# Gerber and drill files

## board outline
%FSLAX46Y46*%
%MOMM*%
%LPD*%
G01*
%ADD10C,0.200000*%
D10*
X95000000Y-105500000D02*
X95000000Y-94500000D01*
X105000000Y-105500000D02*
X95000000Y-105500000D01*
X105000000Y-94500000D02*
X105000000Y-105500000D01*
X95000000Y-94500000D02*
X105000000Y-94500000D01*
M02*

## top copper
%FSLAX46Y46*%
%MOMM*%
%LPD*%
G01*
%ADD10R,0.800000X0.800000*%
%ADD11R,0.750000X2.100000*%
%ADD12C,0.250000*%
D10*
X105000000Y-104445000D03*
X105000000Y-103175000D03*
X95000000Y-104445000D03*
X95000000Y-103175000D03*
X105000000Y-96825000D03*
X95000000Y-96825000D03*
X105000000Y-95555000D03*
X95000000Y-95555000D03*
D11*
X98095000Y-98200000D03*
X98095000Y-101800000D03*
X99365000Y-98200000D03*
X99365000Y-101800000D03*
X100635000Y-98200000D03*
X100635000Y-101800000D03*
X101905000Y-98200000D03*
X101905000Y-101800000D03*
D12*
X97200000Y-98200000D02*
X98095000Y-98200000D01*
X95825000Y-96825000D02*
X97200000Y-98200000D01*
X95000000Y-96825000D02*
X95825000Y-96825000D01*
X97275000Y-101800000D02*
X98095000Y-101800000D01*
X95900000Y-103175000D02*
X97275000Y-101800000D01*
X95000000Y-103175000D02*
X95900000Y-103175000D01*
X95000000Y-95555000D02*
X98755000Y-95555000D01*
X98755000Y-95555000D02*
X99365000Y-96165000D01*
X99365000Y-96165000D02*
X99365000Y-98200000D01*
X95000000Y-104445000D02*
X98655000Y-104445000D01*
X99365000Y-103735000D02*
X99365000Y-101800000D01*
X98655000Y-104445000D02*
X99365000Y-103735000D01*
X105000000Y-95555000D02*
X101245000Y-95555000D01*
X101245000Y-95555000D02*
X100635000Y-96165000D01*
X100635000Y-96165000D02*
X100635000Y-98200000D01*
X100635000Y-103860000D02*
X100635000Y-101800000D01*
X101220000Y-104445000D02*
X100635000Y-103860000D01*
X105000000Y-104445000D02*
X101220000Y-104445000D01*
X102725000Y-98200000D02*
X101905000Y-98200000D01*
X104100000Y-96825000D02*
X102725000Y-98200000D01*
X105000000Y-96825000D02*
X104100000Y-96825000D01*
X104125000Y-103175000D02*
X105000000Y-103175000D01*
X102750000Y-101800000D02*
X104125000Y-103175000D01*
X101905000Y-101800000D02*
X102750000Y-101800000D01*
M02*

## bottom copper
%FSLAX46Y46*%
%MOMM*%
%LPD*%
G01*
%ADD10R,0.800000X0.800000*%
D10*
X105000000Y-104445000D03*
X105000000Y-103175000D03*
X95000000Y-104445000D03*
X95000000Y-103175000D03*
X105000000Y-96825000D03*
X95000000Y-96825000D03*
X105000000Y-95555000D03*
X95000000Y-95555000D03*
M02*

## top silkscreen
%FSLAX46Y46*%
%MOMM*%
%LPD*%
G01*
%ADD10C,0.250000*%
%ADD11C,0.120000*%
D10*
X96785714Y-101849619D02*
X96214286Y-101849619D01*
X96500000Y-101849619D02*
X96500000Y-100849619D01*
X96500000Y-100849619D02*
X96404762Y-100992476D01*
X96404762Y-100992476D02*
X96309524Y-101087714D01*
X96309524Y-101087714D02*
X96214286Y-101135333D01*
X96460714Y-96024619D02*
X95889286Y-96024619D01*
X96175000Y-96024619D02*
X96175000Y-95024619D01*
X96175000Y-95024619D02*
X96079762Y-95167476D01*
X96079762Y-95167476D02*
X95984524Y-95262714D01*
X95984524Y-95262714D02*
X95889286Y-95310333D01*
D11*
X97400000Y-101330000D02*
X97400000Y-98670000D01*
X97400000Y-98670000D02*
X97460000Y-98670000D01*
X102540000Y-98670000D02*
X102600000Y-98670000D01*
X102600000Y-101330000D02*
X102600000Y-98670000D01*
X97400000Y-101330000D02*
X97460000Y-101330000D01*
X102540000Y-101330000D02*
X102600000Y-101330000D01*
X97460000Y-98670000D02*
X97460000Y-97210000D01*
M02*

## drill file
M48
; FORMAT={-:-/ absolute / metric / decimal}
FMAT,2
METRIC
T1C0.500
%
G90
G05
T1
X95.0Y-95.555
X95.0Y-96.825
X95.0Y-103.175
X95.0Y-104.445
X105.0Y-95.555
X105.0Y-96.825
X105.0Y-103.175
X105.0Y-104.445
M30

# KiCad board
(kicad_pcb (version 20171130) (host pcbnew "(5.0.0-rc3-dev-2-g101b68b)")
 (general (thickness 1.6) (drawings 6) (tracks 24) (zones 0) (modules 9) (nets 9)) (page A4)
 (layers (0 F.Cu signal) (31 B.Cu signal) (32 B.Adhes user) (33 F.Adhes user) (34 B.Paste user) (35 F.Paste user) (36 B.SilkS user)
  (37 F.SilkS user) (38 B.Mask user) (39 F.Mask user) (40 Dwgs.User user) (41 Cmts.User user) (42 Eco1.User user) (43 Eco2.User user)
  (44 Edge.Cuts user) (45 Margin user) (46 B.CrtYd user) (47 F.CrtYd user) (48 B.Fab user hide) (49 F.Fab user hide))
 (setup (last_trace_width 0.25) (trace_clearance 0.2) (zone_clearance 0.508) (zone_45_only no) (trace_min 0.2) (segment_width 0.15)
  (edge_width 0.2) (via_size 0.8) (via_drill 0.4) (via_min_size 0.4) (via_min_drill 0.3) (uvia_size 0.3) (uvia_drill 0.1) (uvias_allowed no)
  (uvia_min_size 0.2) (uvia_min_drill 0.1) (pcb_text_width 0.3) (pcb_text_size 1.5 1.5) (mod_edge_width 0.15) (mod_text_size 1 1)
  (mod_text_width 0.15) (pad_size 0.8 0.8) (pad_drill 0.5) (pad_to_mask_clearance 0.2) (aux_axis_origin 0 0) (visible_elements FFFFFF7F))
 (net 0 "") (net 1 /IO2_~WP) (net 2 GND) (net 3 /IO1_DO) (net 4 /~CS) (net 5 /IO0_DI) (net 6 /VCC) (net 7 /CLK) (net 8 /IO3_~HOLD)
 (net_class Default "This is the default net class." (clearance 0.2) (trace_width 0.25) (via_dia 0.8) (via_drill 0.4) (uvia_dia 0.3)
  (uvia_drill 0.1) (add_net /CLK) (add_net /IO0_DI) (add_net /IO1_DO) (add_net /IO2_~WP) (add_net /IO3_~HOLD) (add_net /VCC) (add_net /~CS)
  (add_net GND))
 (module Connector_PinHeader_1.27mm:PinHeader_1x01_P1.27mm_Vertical (layer F.Cu) (at 105 104.445)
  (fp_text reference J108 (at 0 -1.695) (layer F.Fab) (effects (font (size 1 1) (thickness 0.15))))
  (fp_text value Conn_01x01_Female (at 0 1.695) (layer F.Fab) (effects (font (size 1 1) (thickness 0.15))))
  (pad 1 thru_hole rect (at 0 0) (size 0.8 0.8) (drill 0.5) (layers *.Cu *.Mask) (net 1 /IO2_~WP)))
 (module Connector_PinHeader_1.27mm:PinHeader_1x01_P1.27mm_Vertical (layer F.Cu) (at 105 103.175)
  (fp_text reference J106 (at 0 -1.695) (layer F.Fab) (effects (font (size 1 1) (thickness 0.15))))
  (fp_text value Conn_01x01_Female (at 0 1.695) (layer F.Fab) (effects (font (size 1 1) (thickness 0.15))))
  (pad 1 thru_hole rect (at 0 0) (size 0.8 0.8) (drill 0.5) (layers *.Cu *.Mask) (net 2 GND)))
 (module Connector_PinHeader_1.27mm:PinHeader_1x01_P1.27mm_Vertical (layer F.Cu) (at 95 104.445)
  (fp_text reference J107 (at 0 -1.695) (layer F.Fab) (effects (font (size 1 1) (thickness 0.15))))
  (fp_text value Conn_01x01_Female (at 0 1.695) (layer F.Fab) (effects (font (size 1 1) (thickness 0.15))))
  (pad 1 thru_hole rect (at 0 0) (size 0.8 0.8) (drill 0.5) (layers *.Cu *.Mask) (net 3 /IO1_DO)))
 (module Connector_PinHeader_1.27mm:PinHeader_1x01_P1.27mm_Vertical (layer F.Cu) (at 95 103.175)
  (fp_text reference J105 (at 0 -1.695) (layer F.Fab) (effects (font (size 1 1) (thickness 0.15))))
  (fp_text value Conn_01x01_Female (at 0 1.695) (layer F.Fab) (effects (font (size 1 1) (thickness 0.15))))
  (pad 1 thru_hole rect (at 0 0) (size 0.8 0.8) (drill 0.5) (layers *.Cu *.Mask) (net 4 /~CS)))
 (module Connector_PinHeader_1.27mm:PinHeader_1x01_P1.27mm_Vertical (layer F.Cu) (at 105 96.825)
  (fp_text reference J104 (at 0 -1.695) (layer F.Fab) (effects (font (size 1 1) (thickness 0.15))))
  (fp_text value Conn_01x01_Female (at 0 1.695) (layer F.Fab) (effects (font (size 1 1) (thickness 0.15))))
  (pad 1 thru_hole rect (at 0 0) (size 0.8 0.8) (drill 0.5) (layers *.Cu *.Mask) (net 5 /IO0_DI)))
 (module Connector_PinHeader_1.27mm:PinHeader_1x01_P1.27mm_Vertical (layer F.Cu) (at 95 96.825)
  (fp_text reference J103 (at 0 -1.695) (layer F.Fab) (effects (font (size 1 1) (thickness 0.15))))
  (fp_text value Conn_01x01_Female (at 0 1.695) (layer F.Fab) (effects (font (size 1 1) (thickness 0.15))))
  (pad 1 thru_hole rect (at 0 0) (size 0.8 0.8) (drill 0.5) (layers *.Cu *.Mask) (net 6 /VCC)))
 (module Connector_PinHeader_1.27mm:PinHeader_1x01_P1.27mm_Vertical (layer F.Cu) (at 105 95.555)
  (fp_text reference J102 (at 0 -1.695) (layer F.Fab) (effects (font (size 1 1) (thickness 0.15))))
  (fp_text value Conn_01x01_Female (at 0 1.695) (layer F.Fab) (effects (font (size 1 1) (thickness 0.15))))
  (pad 1 thru_hole rect (at 0 0) (size 0.8 0.8) (drill 0.5) (layers *.Cu *.Mask) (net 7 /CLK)))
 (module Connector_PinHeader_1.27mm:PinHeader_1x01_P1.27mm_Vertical (layer F.Cu) (at 95 95.555)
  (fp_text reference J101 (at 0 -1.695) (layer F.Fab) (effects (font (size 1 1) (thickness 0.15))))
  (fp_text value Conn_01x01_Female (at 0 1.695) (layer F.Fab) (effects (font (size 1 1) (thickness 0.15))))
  (pad 1 thru_hole rect (at 0 0) (size 0.8 0.8) (drill 0.5) (layers *.Cu *.Mask) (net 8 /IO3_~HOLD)))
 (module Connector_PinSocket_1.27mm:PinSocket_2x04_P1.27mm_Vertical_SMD (layer F.Cu) (at 100 100 90)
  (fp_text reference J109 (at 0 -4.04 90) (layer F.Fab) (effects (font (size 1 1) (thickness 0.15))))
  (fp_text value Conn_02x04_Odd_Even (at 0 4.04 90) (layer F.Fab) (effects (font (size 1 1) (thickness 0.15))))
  (fp_line (start -1.33 -2.6) (end 1.33 -2.6) (layer F.SilkS) (width 0.12))
  (fp_line (start 1.33 -2.6) (end 1.33 -2.54) (layer F.SilkS) (width 0.12))
  (fp_line (start 1.33 2.54) (end 1.33 2.6) (layer F.SilkS) (width 0.12))
  (fp_line (start -1.33 2.6) (end 1.33 2.6) (layer F.SilkS) (width 0.12))
  (fp_line (start -1.33 -2.6) (end -1.33 -2.54) (layer F.SilkS) (width 0.12))
  (fp_line (start -1.33 2.54) (end -1.33 2.6) (layer F.SilkS) (width 0.12))
  (fp_line (start 1.33 -2.54) (end 2.79 -2.54) (layer F.SilkS) (width 0.12))
  (pad 1 smd rect (at 1.8 -1.905 90) (size 2.1 0.75) (layers F.Cu F.Paste F.Mask) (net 6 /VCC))
  (pad 2 smd rect (at -1.8 -1.905 90) (size 2.1 0.75) (layers F.Cu F.Paste F.Mask) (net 4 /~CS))
  (pad 3 smd rect (at 1.8 -0.635 90) (size 2.1 0.75) (layers F.Cu F.Paste F.Mask) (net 8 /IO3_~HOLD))
  (pad 4 smd rect (at -1.8 -0.635 90) (size 2.1 0.75) (layers F.Cu F.Paste F.Mask) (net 3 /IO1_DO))
  (pad 5 smd rect (at 1.8 0.635 90) (size 2.1 0.75) (layers F.Cu F.Paste F.Mask) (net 7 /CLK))
  (pad 6 smd rect (at -1.8 0.635 90) (size 2.1 0.75) (layers F.Cu F.Paste F.Mask) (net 1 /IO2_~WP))
  (pad 7 smd rect (at 1.8 1.905 90) (size 2.1 0.75) (layers F.Cu F.Paste F.Mask) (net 5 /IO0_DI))
  (pad 8 smd rect (at -1.8 1.905 90) (size 2.1 0.75) (layers F.Cu F.Paste F.Mask) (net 2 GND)))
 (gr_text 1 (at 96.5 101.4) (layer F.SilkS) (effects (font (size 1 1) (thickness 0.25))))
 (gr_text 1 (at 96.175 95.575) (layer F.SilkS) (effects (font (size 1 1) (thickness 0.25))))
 (gr_line (start 95 105.5) (end 95 94.5) (layer Edge.Cuts) (width 0.2))
 (gr_line (start 105 105.5) (end 95 105.5) (layer Edge.Cuts) (width 0.2))
 (gr_line (start 105 94.5) (end 105 105.5) (layer Edge.Cuts) (width 0.2))
 (gr_line (start 95 94.5) (end 105 94.5) (layer Edge.Cuts) (width 0.2))
 (segment (start 97.2 98.2) (end 98.095 98.2) (width 0.25) (layer F.Cu) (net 6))
 (segment (start 95.825 96.825) (end 97.2 98.2) (width 0.25) (layer F.Cu) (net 6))
 (segment (start 95 96.825) (end 95.825 96.825) (width 0.25) (layer F.Cu) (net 6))
 (segment (start 97.275 101.8) (end 98.095 101.8) (width 0.25) (layer F.Cu) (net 4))
 (segment (start 95.9 103.175) (end 97.275 101.8) (width 0.25) (layer F.Cu) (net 4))
 (segment (start 95 103.175) (end 95.9 103.175) (width 0.25) (layer F.Cu) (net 4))
 (segment (start 95 95.555) (end 98.755 95.555) (width 0.25) (layer F.Cu) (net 8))
 (segment (start 98.755 95.555) (end 99.365 96.165) (width 0.25) (layer F.Cu) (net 8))
 (segment (start 99.365 96.165) (end 99.365 98.2) (width 0.25) (layer F.Cu) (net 8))
 (segment (start 95 104.445) (end 98.655 104.445) (width 0.25) (layer F.Cu) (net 3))
 (segment (start 99.365 103.735) (end 99.365 101.8) (width 0.25) (layer F.Cu) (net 3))
 (segment (start 98.655 104.445) (end 99.365 103.735) (width 0.25) (layer F.Cu) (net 3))
 (segment (start 105 95.555) (end 101.245 95.555) (width 0.25) (layer F.Cu) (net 7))
 (segment (start 101.245 95.555) (end 100.635 96.165) (width 0.25) (layer F.Cu) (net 7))
 (segment (start 100.635 96.165) (end 100.635 98.2) (width 0.25) (layer F.Cu) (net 7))
 (segment (start 100.635 103.86) (end 100.635 101.8) (width 0.25) (layer F.Cu) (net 1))
 (segment (start 101.22 104.445) (end 100.635 103.86) (width 0.25) (layer F.Cu) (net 1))
 (segment (start 105 104.445) (end 101.22 104.445) (width 0.25) (layer F.Cu) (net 1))
 (segment (start 102.725 98.2) (end 101.905 98.2) (width 0.25) (layer F.Cu) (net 5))
 (segment (start 104.1 96.825) (end 102.725 98.2) (width 0.25) (layer F.Cu) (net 5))
 (segment (start 105 96.825) (end 104.1 96.825) (width 0.25) (layer F.Cu) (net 5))
 (segment (start 104.125 103.175) (end 105 103.175) (width 0.25) (layer F.Cu) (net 2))
 (segment (start 102.75 101.8) (end 104.125 103.175) (width 0.25) (layer F.Cu) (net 2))
 (segment (start 101.905 101.8) (end 102.75 101.8) (width 0.25) (layer F.Cu) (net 2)))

